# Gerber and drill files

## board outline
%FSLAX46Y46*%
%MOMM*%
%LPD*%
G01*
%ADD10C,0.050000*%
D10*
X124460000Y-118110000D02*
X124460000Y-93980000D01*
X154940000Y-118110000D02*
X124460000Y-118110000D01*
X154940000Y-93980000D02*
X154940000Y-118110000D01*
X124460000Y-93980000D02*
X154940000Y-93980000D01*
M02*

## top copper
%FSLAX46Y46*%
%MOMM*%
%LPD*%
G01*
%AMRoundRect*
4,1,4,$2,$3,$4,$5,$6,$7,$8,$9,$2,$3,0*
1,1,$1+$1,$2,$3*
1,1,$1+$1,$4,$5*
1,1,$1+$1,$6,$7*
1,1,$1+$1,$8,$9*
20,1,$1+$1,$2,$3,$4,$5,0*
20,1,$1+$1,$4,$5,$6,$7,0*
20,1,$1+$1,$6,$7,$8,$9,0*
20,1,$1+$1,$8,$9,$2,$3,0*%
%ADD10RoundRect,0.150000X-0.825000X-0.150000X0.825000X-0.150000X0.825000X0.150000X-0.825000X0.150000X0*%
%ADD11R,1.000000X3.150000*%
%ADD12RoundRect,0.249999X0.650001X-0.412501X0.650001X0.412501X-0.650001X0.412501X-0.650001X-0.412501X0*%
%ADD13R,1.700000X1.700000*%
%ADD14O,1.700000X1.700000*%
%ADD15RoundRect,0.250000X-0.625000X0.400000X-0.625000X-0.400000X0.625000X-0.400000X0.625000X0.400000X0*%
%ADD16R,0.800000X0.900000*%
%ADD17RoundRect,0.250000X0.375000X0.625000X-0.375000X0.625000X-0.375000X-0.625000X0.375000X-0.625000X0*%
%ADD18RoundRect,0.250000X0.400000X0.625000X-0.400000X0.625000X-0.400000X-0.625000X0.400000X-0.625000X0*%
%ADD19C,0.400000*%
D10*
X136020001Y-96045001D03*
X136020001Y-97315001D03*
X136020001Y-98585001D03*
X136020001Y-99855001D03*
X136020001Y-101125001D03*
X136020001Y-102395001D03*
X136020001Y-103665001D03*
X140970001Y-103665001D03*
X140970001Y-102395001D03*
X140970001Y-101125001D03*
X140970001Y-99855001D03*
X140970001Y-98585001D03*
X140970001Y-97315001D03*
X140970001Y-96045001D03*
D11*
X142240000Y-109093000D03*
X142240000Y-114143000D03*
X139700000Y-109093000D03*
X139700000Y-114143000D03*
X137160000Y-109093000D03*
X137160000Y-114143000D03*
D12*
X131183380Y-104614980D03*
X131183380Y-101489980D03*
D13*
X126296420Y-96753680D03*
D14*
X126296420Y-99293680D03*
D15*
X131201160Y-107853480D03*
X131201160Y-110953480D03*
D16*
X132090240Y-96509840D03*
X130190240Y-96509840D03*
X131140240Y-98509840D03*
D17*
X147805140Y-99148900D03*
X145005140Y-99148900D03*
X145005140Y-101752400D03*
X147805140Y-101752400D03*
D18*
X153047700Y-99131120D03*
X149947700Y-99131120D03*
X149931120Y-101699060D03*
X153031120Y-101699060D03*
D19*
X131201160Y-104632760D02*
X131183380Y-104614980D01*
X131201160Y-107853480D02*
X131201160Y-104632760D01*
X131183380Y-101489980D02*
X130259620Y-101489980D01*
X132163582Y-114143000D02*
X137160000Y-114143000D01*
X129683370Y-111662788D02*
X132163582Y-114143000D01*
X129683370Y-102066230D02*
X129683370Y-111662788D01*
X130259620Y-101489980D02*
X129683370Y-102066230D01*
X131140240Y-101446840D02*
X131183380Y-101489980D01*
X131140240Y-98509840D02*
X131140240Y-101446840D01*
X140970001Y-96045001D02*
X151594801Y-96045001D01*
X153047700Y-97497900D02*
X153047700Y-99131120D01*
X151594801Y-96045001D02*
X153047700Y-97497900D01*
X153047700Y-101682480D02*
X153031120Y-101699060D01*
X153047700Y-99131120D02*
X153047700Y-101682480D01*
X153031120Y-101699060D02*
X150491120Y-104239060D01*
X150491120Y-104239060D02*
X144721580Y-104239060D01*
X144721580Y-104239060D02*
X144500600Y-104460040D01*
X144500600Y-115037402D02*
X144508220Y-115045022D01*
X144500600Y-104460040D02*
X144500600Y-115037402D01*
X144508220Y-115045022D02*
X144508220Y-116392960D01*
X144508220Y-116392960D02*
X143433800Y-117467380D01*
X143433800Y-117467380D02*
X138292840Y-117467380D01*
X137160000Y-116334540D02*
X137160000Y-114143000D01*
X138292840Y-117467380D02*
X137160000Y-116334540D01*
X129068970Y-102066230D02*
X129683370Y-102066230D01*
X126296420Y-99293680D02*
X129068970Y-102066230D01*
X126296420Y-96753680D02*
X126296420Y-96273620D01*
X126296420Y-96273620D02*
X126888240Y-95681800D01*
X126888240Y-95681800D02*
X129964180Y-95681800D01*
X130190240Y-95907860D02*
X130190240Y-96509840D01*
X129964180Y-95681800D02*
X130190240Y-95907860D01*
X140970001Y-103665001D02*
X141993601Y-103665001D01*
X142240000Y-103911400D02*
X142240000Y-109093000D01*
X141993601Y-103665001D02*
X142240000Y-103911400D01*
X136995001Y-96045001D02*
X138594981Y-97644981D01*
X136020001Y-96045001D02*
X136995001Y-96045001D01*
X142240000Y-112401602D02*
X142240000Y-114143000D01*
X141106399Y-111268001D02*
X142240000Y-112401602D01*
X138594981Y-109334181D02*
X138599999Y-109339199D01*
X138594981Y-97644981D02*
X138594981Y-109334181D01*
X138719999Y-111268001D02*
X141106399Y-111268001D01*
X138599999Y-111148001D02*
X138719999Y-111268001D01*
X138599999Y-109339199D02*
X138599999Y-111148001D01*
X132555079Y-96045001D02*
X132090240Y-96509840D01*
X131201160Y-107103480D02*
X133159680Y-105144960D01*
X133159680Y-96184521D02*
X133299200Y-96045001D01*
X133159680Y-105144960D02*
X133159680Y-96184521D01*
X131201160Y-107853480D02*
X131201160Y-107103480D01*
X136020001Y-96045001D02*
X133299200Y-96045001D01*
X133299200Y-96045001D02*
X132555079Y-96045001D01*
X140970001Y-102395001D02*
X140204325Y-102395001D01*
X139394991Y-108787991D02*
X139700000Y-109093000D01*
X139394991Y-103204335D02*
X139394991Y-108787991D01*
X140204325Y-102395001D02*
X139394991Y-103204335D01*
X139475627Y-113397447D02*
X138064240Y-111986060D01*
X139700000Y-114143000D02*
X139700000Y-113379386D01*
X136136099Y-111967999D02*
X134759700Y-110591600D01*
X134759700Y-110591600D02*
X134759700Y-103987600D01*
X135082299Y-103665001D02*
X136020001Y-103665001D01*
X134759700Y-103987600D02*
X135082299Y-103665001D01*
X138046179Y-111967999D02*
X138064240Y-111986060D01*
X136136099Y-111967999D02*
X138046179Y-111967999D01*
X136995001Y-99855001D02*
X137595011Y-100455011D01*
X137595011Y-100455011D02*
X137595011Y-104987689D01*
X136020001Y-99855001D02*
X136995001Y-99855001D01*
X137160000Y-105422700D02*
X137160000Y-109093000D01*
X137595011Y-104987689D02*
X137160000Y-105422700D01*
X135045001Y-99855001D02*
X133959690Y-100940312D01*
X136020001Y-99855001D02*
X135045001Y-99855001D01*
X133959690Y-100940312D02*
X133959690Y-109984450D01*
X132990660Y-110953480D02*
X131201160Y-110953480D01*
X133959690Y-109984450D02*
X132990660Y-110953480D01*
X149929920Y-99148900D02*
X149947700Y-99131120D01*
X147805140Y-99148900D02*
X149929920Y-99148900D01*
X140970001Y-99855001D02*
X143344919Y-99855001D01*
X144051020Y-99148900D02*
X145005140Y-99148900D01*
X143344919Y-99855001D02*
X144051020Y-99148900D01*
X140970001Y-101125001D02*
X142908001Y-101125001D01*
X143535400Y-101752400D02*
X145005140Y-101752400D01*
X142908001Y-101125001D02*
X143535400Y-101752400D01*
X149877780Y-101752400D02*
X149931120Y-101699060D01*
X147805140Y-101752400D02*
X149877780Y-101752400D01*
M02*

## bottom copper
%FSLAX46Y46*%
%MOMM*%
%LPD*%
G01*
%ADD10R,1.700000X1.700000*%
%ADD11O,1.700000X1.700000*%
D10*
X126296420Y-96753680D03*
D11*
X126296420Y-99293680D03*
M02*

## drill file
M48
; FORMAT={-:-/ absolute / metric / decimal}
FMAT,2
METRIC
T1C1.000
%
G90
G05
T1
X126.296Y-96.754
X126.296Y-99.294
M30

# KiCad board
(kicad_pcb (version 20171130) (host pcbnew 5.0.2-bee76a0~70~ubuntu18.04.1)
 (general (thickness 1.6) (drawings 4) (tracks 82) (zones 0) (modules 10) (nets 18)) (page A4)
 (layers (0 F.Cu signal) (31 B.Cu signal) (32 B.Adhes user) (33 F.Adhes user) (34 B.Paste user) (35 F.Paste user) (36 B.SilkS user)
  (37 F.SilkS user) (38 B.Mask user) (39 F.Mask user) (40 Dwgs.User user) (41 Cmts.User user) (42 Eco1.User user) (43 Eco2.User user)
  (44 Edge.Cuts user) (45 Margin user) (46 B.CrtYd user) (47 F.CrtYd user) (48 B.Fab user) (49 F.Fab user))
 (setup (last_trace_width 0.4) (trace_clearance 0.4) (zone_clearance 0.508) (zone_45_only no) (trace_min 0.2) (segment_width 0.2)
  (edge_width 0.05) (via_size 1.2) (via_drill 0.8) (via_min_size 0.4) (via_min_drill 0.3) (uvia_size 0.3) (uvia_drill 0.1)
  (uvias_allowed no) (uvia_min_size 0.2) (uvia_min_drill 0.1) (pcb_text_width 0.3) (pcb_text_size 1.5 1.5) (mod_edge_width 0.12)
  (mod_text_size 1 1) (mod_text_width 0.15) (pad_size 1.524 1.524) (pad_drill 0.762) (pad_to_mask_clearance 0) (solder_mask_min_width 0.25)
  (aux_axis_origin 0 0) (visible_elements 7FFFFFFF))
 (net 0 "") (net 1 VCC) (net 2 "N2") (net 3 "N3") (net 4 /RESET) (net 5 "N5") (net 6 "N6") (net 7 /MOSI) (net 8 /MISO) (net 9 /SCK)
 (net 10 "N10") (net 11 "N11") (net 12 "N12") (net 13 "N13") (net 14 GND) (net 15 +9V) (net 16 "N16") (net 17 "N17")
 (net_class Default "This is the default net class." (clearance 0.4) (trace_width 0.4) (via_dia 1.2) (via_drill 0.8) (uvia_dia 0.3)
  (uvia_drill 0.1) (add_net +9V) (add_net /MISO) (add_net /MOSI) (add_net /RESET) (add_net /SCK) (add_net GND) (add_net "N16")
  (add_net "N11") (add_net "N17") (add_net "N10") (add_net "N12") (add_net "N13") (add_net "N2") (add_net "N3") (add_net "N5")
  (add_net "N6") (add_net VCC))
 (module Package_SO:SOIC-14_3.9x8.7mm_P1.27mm (layer F.Cu) (at 138.495001 99.855001)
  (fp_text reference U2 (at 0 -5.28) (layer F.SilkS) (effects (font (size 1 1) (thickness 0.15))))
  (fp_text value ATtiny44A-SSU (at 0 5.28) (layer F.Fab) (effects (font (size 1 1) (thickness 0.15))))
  (pad 1 smd roundrect (at -2.475 -3.81) (size 1.95 0.6) (layers F.Cu F.Paste F.Mask) (roundrect_rratio 0.25) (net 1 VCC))
  (pad 2 smd roundrect (at -2.475 -2.54) (size 1.95 0.6) (layers F.Cu F.Paste F.Mask) (roundrect_rratio 0.25) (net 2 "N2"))
  (pad 3 smd roundrect (at -2.475 -1.27) (size 1.95 0.6) (layers F.Cu F.Paste F.Mask) (roundrect_rratio 0.25) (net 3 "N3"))
  (pad 4 smd roundrect (at -2.475 0) (size 1.95 0.6) (layers F.Cu F.Paste F.Mask) (roundrect_rratio 0.25) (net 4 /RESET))
  (pad 5 smd roundrect (at -2.475 1.27) (size 1.95 0.6) (layers F.Cu F.Paste F.Mask) (roundrect_rratio 0.25) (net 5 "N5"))
  (pad 6 smd roundrect (at -2.475 2.54) (size 1.95 0.6) (layers F.Cu F.Paste F.Mask) (roundrect_rratio 0.25) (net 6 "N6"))
  (pad 7 smd roundrect (at -2.475 3.81) (size 1.95 0.6) (layers F.Cu F.Paste F.Mask) (roundrect_rratio 0.25) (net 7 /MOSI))
  (pad 8 smd roundrect (at 2.475 3.81) (size 1.95 0.6) (layers F.Cu F.Paste F.Mask) (roundrect_rratio 0.25) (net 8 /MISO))
  (pad 9 smd roundrect (at 2.475 2.54) (size 1.95 0.6) (layers F.Cu F.Paste F.Mask) (roundrect_rratio 0.25) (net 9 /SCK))
  (pad 10 smd roundrect (at 2.475 1.27) (size 1.95 0.6) (layers F.Cu F.Paste F.Mask) (roundrect_rratio 0.25) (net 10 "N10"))
  (pad 11 smd roundrect (at 2.475 0) (size 1.95 0.6) (layers F.Cu F.Paste F.Mask) (roundrect_rratio 0.25) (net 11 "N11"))
  (pad 12 smd roundrect (at 2.475 -1.27) (size 1.95 0.6) (layers F.Cu F.Paste F.Mask) (roundrect_rratio 0.25) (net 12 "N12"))
  (pad 13 smd roundrect (at 2.475 -2.54) (size 1.95 0.6) (layers F.Cu F.Paste F.Mask) (roundrect_rratio 0.25) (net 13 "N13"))
  (pad 14 smd roundrect (at 2.475 -3.81) (size 1.95 0.6) (layers F.Cu F.Paste F.Mask) (roundrect_rratio 0.25) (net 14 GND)))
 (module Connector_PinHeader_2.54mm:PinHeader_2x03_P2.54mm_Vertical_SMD (layer F.Cu) (at 139.7 111.618 270)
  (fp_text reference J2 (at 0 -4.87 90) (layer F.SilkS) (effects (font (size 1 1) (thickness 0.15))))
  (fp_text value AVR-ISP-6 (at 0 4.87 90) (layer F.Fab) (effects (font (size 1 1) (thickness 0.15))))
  (pad 1 smd rect (at -2.525 -2.54 270) (size 3.15 1) (layers F.Cu F.Paste F.Mask) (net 8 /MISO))
  (pad 2 smd rect (at 2.525 -2.54 270) (size 3.15 1) (layers F.Cu F.Paste F.Mask) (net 1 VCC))
  (pad 3 smd rect (at -2.525 0 270) (size 3.15 1) (layers F.Cu F.Paste F.Mask) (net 9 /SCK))
  (pad 4 smd rect (at 2.525 0 270) (size 3.15 1) (layers F.Cu F.Paste F.Mask) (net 7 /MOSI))
  (pad 5 smd rect (at -2.525 2.54 270) (size 3.15 1) (layers F.Cu F.Paste F.Mask) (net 4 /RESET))
  (pad 6 smd rect (at 2.525 2.54 270) (size 3.15 1) (layers F.Cu F.Paste F.Mask) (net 14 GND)))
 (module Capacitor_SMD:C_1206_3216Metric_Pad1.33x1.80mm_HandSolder (layer F.Cu) (at 131.18338 103.05248 90)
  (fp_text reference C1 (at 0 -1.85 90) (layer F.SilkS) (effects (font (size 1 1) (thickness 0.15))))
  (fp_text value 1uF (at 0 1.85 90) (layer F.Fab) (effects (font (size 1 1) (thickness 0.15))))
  (pad 1 smd roundrect (at -1.5625 0 90) (size 1.325 1.8) (layers F.Cu F.Paste F.Mask) (roundrect_rratio 0.1886784905660377) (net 1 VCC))
  (pad 2 smd roundrect (at 1.5625 0 90) (size 1.325 1.8) (layers F.Cu F.Paste F.Mask) (roundrect_rratio 0.1886784905660377) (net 14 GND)))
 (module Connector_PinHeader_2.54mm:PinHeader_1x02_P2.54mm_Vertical (layer F.Cu) (at 126.29642 96.75368)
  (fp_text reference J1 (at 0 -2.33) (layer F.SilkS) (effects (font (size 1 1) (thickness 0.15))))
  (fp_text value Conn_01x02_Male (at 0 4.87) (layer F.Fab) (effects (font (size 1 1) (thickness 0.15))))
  (pad 1 thru_hole rect (at 0 0) (size 1.7 1.7) (drill 1) (layers *.Cu *.Mask) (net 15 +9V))
  (pad 2 thru_hole oval (at 0 2.54) (size 1.7 1.7) (drill 1) (layers *.Cu *.Mask) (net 14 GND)))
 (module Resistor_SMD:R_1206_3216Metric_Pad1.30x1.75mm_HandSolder (layer F.Cu) (at 131.20116 109.40348 270)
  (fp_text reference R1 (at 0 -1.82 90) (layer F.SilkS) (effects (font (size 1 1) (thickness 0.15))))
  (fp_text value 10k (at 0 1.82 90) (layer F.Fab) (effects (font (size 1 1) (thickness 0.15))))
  (pad 1 smd roundrect (at -1.55 0 270) (size 1.3 1.75) (layers F.Cu F.Paste F.Mask) (roundrect_rratio 0.1923076923076923) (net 1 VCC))
  (pad 2 smd roundrect (at 1.55 0 270) (size 1.3 1.75) (layers F.Cu F.Paste F.Mask) (roundrect_rratio 0.1923076923076923) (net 4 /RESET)))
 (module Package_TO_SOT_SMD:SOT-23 (layer F.Cu) (at 131.14024 97.50984 270)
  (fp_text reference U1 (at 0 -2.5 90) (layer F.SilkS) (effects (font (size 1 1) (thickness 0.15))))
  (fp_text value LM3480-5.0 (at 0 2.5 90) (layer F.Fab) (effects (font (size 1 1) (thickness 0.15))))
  (pad 1 smd rect (at -1 -0.95 270) (size 0.9 0.8) (layers F.Cu F.Paste F.Mask) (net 1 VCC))
  (pad 2 smd rect (at -1 0.95 270) (size 0.9 0.8) (layers F.Cu F.Paste F.Mask) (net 15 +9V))
  (pad 3 smd rect (at 1 0 270) (size 0.9 0.8) (layers F.Cu F.Paste F.Mask) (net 14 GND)))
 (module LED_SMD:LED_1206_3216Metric (layer F.Cu) (at 146.40514 99.1489 180)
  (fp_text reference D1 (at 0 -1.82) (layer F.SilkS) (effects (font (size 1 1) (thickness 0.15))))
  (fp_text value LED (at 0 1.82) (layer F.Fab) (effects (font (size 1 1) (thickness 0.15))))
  (pad 1 smd roundrect (at -1.4 0 180) (size 1.25 1.75) (layers F.Cu F.Paste F.Mask) (roundrect_rratio 0.2) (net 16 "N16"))
  (pad 2 smd roundrect (at 1.4 0 180) (size 1.25 1.75) (layers F.Cu F.Paste F.Mask) (roundrect_rratio 0.2) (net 11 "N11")))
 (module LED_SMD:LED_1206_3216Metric (layer F.Cu) (at 146.40514 101.7524 180)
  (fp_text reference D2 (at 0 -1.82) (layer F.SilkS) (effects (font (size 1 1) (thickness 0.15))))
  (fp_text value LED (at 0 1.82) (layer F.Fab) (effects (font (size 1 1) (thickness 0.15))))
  (pad 2 smd roundrect (at 1.4 0 180) (size 1.25 1.75) (layers F.Cu F.Paste F.Mask) (roundrect_rratio 0.2) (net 10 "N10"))
  (pad 1 smd roundrect (at -1.4 0 180) (size 1.25 1.75) (layers F.Cu F.Paste F.Mask) (roundrect_rratio 0.2) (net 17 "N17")))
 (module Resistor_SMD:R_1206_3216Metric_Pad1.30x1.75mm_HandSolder (layer F.Cu) (at 151.4977 99.13112 180)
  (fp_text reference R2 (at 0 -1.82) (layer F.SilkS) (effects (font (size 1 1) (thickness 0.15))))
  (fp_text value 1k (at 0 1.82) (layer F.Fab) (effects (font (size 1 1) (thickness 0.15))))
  (pad 1 smd roundrect (at -1.55 0 180) (size 1.3 1.75) (layers F.Cu F.Paste F.Mask) (roundrect_rratio 0.1923076923076923) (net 14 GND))
  (pad 2 smd roundrect (at 1.55 0 180) (size 1.3 1.75) (layers F.Cu F.Paste F.Mask) (roundrect_rratio 0.1923076923076923) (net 16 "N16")))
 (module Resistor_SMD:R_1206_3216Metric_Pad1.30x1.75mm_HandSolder (layer F.Cu) (at 151.48112 101.69906 180)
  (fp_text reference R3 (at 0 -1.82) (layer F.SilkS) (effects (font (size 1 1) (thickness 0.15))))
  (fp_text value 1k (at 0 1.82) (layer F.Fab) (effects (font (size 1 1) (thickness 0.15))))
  (pad 2 smd roundrect (at 1.55 0 180) (size 1.3 1.75) (layers F.Cu F.Paste F.Mask) (roundrect_rratio 0.1923076923076923) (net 17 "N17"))
  (pad 1 smd roundrect (at -1.55 0 180) (size 1.3 1.75) (layers F.Cu F.Paste F.Mask) (roundrect_rratio 0.1923076923076923) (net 14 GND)))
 (gr_line (start 124.46 118.11) (end 124.46 93.98) (layer Edge.Cuts) (width 0.05))
 (gr_line (start 154.94 118.11) (end 124.46 118.11) (layer Edge.Cuts) (width 0.05))
 (gr_line (start 154.94 93.98) (end 154.94 118.11) (layer Edge.Cuts) (width 0.05))
 (gr_line (start 124.46 93.98) (end 154.94 93.98) (layer Edge.Cuts) (width 0.05))
 (segment (start 131.20116 104.63276) (end 131.18338 104.61498) (width 0.4) (layer F.Cu) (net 1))
 (segment (start 131.20116 107.85348) (end 131.20116 104.63276) (width 0.4) (layer F.Cu) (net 1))
 (segment (start 131.18338 101.48998) (end 130.25962 101.48998) (width 0.4) (layer F.Cu) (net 14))
 (segment (start 132.163582 114.143) (end 137.16 114.143) (width 0.4) (layer F.Cu) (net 14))
 (segment (start 129.68337 111.662788) (end 132.163582 114.143) (width 0.4) (layer F.Cu) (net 14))
 (segment (start 129.68337 102.06623) (end 129.68337 111.662788) (width 0.4) (layer F.Cu) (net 14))
 (segment (start 130.25962 101.48998) (end 129.68337 102.06623) (width 0.4) (layer F.Cu) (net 14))
 (segment (start 131.14024 101.44684) (end 131.18338 101.48998) (width 0.4) (layer F.Cu) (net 14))
 (segment (start 131.14024 98.50984) (end 131.14024 101.44684) (width 0.4) (layer F.Cu) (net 14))
 (segment (start 140.970001 96.045001) (end 151.594801 96.045001) (width 0.4) (layer F.Cu) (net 14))
 (segment (start 153.0477 97.4979) (end 153.0477 99.13112) (width 0.4) (layer F.Cu) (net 14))
 (segment (start 151.594801 96.045001) (end 153.0477 97.4979) (width 0.4) (layer F.Cu) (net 14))
 (segment (start 153.0477 101.68248) (end 153.03112 101.69906) (width 0.4) (layer F.Cu) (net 14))
 (segment (start 153.0477 99.13112) (end 153.0477 101.68248) (width 0.4) (layer F.Cu) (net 14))
 (segment (start 153.03112 101.69906) (end 150.49112 104.23906) (width 0.4) (layer F.Cu) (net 14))
 (segment (start 150.49112 104.23906) (end 144.72158 104.23906) (width 0.4) (layer F.Cu) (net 14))
 (segment (start 144.72158 104.23906) (end 144.5006 104.46004) (width 0.4) (layer F.Cu) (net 14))
 (segment (start 144.5006 115.037402) (end 144.50822 115.045022) (width 0.4) (layer F.Cu) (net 14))
 (segment (start 144.5006 104.46004) (end 144.5006 115.037402) (width 0.4) (layer F.Cu) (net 14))
 (segment (start 144.50822 115.045022) (end 144.50822 116.39296) (width 0.4) (layer F.Cu) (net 14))
 (segment (start 144.50822 116.39296) (end 143.4338 117.46738) (width 0.4) (layer F.Cu) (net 14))
 (segment (start 143.4338 117.46738) (end 138.29284 117.46738) (width 0.4) (layer F.Cu) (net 14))
 (segment (start 137.16 116.33454) (end 137.16 114.143) (width 0.4) (layer F.Cu) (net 14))
 (segment (start 138.29284 117.46738) (end 137.16 116.33454) (width 0.4) (layer F.Cu) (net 14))
 (segment (start 129.06897 102.06623) (end 129.68337 102.06623) (width 0.4) (layer F.Cu) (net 14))
 (segment (start 126.29642 99.29368) (end 129.06897 102.06623) (width 0.4) (layer F.Cu) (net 14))
 (segment (start 126.29642 96.75368) (end 126.29642 96.27362) (width 0.4) (layer F.Cu) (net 15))
 (segment (start 126.29642 96.27362) (end 126.88824 95.6818) (width 0.4) (layer F.Cu) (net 15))
 (segment (start 126.88824 95.6818) (end 129.96418 95.6818) (width 0.4) (layer F.Cu) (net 15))
 (segment (start 130.19024 95.90786) (end 130.19024 96.50984) (width 0.4) (layer F.Cu) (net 15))
 (segment (start 129.96418 95.6818) (end 130.19024 95.90786) (width 0.4) (layer F.Cu) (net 15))
 (segment (start 140.970001 103.665001) (end 141.993601 103.665001) (width 0.4) (layer F.Cu) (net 8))
 (segment (start 142.24 103.9114) (end 142.24 109.093) (width 0.4) (layer F.Cu) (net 8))
 (segment (start 141.993601 103.665001) (end 142.24 103.9114) (width 0.4) (layer F.Cu) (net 8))
 (segment (start 136.995001 96.045001) (end 138.594981 97.644981) (width 0.4) (layer F.Cu) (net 1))
 (segment (start 136.020001 96.045001) (end 136.995001 96.045001) (width 0.4) (layer F.Cu) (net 1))
 (segment (start 142.24 112.401602) (end 142.24 114.143) (width 0.4) (layer F.Cu) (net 1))
 (segment (start 141.106399 111.268001) (end 142.24 112.401602) (width 0.4) (layer F.Cu) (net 1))
 (segment (start 138.594981 109.334181) (end 138.599999 109.339199) (width 0.4) (layer F.Cu) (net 1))
 (segment (start 138.594981 97.644981) (end 138.594981 109.334181) (width 0.4) (layer F.Cu) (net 1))
 (segment (start 138.719999 111.268001) (end 141.106399 111.268001) (width 0.4) (layer F.Cu) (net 1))
 (segment (start 138.599999 111.148001) (end 138.719999 111.268001) (width 0.4) (layer F.Cu) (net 1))
 (segment (start 138.599999 109.339199) (end 138.599999 111.148001) (width 0.4) (layer F.Cu) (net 1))
 (segment (start 132.555079 96.045001) (end 132.09024 96.50984) (width 0.4) (layer F.Cu) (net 1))
 (segment (start 131.20116 107.10348) (end 133.15968 105.14496) (width 0.4) (layer F.Cu) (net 1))
 (segment (start 133.15968 96.184521) (end 133.2992 96.045001) (width 0.4) (layer F.Cu) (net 1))
 (segment (start 133.15968 105.14496) (end 133.15968 96.184521) (width 0.4) (layer F.Cu) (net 1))
 (segment (start 131.20116 107.85348) (end 131.20116 107.10348) (width 0.4) (layer F.Cu) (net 1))
 (segment (start 136.020001 96.045001) (end 133.2992 96.045001) (width 0.4) (layer F.Cu) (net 1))
 (segment (start 133.2992 96.045001) (end 132.555079 96.045001) (width 0.4) (layer F.Cu) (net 1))
 (segment (start 140.970001 102.395001) (end 140.204325 102.395001) (width 0.4) (layer F.Cu) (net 9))
 (segment (start 139.394991 108.787991) (end 139.7 109.093) (width 0.4) (layer F.Cu) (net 9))
 (segment (start 139.394991 103.204335) (end 139.394991 108.787991) (width 0.4) (layer F.Cu) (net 9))
 (segment (start 140.204325 102.395001) (end 139.394991 103.204335) (width 0.4) (layer F.Cu) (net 9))
 (segment (start 139.475627 113.397447) (end 138.06424 111.98606) (width 0.4) (layer F.Cu) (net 7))
 (segment (start 139.7 114.143) (end 139.7 113.379386) (width 0.4) (layer F.Cu) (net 7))
 (segment (start 136.136099 111.967999) (end 134.7597 110.5916) (width 0.4) (layer F.Cu) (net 7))
 (segment (start 134.7597 110.5916) (end 134.7597 103.9876) (width 0.4) (layer F.Cu) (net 7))
 (segment (start 135.082299 103.665001) (end 136.020001 103.665001) (width 0.4) (layer F.Cu) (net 7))
 (segment (start 134.7597 103.9876) (end 135.082299 103.665001) (width 0.4) (layer F.Cu) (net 7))
 (segment (start 138.046179 111.967999) (end 138.06424 111.98606) (width 0.4) (layer F.Cu) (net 7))
 (segment (start 136.136099 111.967999) (end 138.046179 111.967999) (width 0.4) (layer F.Cu) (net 7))
 (segment (start 136.995001 99.855001) (end 137.595011 100.455011) (width 0.4) (layer F.Cu) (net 4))
 (segment (start 137.595011 100.455011) (end 137.595011 104.987689) (width 0.4) (layer F.Cu) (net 4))
 (segment (start 136.020001 99.855001) (end 136.995001 99.855001) (width 0.4) (layer F.Cu) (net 4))
 (segment (start 137.16 105.4227) (end 137.16 109.093) (width 0.4) (layer F.Cu) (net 4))
 (segment (start 137.595011 104.987689) (end 137.16 105.4227) (width 0.4) (layer F.Cu) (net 4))
 (segment (start 135.045001 99.855001) (end 133.95969 100.940312) (width 0.4) (layer F.Cu) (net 4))
 (segment (start 136.020001 99.855001) (end 135.045001 99.855001) (width 0.4) (layer F.Cu) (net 4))
 (segment (start 133.95969 100.940312) (end 133.95969 109.98445) (width 0.4) (layer F.Cu) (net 4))
 (segment (start 132.99066 110.95348) (end 131.20116 110.95348) (width 0.4) (layer F.Cu) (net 4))
 (segment (start 133.95969 109.98445) (end 132.99066 110.95348) (width 0.4) (layer F.Cu) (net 4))
 (segment (start 149.92992 99.1489) (end 149.9477 99.13112) (width 0.4) (layer F.Cu) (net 16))
 (segment (start 147.80514 99.1489) (end 149.92992 99.1489) (width 0.4) (layer F.Cu) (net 16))
 (segment (start 140.970001 99.855001) (end 143.344919 99.855001) (width 0.4) (layer F.Cu) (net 11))
 (segment (start 144.05102 99.1489) (end 145.00514 99.1489) (width 0.4) (layer F.Cu) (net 11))
 (segment (start 143.344919 99.855001) (end 144.05102 99.1489) (width 0.4) (layer F.Cu) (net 11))
 (segment (start 140.970001 101.125001) (end 142.908001 101.125001) (width 0.4) (layer F.Cu) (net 10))
 (segment (start 143.5354 101.7524) (end 145.00514 101.7524) (width 0.4) (layer F.Cu) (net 10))
 (segment (start 142.908001 101.125001) (end 143.5354 101.7524) (width 0.4) (layer F.Cu) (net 10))
 (segment (start 149.87778 101.7524) (end 149.93112 101.69906) (width 0.4) (layer F.Cu) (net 17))
 (segment (start 147.80514 101.7524) (end 149.87778 101.7524) (width 0.4) (layer F.Cu) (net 17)))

